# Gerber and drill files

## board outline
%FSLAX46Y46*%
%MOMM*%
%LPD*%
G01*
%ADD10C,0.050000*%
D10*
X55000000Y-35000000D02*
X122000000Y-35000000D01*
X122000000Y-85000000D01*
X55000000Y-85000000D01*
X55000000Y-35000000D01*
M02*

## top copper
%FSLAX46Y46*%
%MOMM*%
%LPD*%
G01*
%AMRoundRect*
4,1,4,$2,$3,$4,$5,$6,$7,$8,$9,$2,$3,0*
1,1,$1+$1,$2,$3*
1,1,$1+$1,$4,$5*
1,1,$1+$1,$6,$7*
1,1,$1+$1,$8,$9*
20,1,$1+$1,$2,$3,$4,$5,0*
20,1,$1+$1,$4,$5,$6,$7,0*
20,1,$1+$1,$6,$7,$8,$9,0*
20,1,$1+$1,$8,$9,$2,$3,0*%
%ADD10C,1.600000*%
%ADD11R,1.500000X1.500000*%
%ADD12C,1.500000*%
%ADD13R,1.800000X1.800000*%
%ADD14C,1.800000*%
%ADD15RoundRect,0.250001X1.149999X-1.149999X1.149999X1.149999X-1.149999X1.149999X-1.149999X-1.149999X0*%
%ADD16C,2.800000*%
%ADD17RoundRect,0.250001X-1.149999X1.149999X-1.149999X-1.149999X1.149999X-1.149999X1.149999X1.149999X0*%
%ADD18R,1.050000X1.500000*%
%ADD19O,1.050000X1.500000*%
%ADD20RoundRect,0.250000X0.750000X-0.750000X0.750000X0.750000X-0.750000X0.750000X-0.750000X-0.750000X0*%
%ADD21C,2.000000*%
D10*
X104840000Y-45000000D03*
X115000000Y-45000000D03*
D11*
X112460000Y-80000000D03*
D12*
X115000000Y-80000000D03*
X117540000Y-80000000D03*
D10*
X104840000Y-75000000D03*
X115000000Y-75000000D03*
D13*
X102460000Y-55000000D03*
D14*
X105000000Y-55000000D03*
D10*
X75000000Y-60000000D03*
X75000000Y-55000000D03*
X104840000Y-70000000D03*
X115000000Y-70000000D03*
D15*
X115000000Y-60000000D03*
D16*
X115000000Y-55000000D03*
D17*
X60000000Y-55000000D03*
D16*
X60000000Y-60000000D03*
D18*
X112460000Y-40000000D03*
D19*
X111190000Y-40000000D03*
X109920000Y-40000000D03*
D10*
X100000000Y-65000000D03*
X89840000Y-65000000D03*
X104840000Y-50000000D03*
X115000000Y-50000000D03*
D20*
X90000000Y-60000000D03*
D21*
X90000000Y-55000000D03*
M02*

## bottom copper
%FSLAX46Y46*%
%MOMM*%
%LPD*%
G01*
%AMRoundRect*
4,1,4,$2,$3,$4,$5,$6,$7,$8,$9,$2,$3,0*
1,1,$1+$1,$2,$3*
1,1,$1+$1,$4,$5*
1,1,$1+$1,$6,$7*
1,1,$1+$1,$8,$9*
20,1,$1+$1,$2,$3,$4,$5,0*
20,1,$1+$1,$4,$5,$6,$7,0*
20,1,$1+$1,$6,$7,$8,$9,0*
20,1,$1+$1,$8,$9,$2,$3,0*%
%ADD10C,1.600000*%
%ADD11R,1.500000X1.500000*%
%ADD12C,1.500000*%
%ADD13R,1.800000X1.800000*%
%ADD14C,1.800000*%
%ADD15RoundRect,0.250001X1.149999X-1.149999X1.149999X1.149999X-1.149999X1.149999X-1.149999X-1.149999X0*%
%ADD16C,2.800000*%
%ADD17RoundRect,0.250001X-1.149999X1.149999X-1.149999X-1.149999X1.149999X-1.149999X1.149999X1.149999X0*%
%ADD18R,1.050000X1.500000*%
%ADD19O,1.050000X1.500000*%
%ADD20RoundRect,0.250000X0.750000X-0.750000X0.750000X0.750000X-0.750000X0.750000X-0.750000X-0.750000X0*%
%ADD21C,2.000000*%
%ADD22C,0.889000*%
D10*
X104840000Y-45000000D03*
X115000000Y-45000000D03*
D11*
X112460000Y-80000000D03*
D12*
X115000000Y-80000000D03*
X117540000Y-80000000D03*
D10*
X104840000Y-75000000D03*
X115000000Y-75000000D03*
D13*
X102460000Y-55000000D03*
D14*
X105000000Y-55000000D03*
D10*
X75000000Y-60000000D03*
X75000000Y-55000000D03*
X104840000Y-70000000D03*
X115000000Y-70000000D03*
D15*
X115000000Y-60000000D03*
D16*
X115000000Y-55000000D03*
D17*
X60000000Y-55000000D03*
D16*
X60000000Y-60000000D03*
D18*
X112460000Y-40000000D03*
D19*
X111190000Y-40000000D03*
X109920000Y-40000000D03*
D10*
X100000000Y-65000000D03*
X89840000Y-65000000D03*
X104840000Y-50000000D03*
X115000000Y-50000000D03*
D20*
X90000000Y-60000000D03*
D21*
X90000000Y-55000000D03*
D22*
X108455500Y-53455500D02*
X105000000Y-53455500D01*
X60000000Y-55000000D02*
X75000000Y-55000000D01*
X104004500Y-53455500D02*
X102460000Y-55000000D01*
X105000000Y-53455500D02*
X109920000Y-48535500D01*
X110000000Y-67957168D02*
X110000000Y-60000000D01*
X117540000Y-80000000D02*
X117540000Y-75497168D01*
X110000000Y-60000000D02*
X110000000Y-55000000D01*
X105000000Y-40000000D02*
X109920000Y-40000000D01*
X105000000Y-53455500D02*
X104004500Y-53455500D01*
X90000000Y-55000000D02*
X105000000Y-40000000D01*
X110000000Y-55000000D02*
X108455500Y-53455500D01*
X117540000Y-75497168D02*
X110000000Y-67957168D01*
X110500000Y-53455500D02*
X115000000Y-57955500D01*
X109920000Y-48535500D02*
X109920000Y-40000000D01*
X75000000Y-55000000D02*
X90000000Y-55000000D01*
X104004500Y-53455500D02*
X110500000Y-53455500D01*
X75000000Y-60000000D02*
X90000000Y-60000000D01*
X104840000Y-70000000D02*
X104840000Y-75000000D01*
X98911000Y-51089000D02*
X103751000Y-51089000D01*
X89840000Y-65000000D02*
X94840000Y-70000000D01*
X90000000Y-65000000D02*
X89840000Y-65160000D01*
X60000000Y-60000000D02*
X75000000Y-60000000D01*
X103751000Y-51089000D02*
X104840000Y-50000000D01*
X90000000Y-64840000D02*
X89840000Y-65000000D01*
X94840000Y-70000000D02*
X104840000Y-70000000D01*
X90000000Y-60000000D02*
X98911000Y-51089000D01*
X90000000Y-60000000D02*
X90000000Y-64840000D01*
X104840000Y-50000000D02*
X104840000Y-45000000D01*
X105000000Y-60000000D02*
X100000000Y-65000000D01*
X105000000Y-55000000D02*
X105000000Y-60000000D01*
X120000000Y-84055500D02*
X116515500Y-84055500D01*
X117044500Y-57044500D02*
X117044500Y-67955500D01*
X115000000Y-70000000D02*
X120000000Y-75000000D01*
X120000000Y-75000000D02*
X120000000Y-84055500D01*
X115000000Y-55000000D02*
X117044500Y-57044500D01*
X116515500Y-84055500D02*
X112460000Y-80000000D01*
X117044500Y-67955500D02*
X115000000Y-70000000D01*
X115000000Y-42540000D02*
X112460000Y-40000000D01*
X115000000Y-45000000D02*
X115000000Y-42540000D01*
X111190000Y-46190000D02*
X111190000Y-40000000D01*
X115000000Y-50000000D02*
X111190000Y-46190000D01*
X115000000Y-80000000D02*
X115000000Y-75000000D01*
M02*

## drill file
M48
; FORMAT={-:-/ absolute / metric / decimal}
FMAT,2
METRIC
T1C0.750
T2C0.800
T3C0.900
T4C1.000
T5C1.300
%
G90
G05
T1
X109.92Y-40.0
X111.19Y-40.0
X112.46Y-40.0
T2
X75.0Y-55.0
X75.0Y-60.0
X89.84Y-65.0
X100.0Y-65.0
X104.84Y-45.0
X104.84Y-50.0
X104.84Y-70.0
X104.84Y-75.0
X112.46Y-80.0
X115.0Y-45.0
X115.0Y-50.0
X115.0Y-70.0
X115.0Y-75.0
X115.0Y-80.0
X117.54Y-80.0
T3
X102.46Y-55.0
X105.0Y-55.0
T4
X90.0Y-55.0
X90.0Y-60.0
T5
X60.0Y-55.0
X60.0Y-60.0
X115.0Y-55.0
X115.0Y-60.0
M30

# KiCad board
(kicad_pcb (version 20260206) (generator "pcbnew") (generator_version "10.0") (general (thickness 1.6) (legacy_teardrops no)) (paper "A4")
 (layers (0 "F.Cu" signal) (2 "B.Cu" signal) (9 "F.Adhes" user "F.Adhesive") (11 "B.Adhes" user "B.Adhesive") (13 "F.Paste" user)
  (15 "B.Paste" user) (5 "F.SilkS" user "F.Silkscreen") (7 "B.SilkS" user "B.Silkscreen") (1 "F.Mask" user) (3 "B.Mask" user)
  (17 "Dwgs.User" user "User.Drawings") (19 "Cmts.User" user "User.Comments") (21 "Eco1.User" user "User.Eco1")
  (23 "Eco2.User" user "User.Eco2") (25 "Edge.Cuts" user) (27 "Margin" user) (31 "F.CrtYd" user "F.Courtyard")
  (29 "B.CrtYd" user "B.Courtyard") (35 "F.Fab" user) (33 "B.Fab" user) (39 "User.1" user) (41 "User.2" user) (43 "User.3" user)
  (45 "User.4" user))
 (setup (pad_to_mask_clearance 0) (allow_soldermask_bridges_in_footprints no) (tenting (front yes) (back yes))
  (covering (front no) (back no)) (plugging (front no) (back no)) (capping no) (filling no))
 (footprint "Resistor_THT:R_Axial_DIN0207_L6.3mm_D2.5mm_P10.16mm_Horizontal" (layer "F.Cu") (at 104.84 45)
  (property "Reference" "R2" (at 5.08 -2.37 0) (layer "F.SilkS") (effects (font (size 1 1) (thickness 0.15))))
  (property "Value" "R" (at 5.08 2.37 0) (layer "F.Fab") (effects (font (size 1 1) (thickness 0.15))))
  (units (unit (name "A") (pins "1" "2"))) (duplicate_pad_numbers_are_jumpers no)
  (pad "1" thru_hole circle (at 0 0) (size 1.6 1.6) (drill 0.8) (layers "*.Cu" "*.Mask") (remove_unused_layers no) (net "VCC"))
  (pad "2" thru_hole circle (at 10.16 0) (size 1.6 1.6) (drill 0.8) (layers "*.Cu" "*.Mask") (remove_unused_layers no) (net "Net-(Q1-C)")))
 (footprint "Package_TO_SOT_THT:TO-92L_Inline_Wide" (layer "F.Cu") (at 112.46 80)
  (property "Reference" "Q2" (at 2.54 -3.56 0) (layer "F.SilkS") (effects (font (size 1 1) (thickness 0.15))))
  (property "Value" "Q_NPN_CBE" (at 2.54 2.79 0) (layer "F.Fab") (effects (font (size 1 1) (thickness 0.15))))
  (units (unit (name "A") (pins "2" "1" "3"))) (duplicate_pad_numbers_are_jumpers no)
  (pad "1" thru_hole rect (at 0 0) (size 1.5 1.5) (drill 0.8) (layers "*.Cu" "*.Mask") (remove_unused_layers no) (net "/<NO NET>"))
  (pad "2" thru_hole circle (at 2.54 0) (size 1.5 1.5) (drill 0.8) (layers "*.Cu" "*.Mask") (remove_unused_layers no) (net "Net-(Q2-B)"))
  (pad "3" thru_hole circle (at 5.08 0) (size 1.5 1.5) (drill 0.8) (layers "*.Cu" "*.Mask") (remove_unused_layers no) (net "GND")))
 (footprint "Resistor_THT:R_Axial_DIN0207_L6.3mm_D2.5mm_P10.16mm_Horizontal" (layer "F.Cu") (at 104.84 75)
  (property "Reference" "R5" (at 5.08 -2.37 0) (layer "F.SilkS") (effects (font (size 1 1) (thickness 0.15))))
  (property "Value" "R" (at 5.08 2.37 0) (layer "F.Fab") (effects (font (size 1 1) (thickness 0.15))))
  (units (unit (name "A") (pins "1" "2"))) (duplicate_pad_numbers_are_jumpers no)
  (pad "1" thru_hole circle (at 0 0) (size 1.6 1.6) (drill 0.8) (layers "*.Cu" "*.Mask") (remove_unused_layers no) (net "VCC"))
  (pad "2" thru_hole circle (at 10.16 0) (size 1.6 1.6) (drill 0.8) (layers "*.Cu" "*.Mask") (remove_unused_layers no) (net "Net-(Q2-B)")))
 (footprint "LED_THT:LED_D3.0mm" (layer "F.Cu") (at 102.46 55)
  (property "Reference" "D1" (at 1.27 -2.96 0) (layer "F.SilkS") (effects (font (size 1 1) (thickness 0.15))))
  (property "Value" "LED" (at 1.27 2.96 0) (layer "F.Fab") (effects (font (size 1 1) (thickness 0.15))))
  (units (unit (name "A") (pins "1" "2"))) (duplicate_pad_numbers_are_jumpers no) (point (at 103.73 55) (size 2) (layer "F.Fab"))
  (pad "1" thru_hole rect (at 0 0) (size 1.8 1.8) (drill 0.9) (layers "*.Cu" "*.Mask") (remove_unused_layers no) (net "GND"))
  (pad "2" thru_hole circle (at 2.54 0) (size 1.8 1.8) (drill 0.9) (layers "*.Cu" "*.Mask") (remove_unused_layers no) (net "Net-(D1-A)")))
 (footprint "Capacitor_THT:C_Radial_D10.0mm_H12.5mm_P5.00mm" (layer "F.Cu") (at 75 60 90)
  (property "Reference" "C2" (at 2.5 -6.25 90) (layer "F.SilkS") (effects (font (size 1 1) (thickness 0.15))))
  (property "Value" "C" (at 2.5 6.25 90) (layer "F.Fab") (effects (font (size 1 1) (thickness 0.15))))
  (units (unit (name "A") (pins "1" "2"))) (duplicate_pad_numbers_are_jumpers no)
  (pad "1" thru_hole circle (at 0 0 90) (size 1.6 1.6) (drill 0.8) (layers "*.Cu" "*.Mask") (remove_unused_layers no) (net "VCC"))
  (pad "2" thru_hole circle (at 5 0 90) (size 1.6 1.6) (drill 0.8) (layers "*.Cu" "*.Mask") (remove_unused_layers no) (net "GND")))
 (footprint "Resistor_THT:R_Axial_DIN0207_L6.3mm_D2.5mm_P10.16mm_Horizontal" (layer "F.Cu") (at 104.84 70)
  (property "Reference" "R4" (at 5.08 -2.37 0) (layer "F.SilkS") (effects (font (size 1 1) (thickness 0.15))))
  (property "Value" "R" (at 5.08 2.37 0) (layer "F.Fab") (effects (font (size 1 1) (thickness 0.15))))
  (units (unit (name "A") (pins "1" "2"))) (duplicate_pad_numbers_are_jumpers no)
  (pad "1" thru_hole circle (at 0 0) (size 1.6 1.6) (drill 0.8) (layers "*.Cu" "*.Mask") (remove_unused_layers no) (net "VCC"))
  (pad "2" thru_hole circle (at 10.16 0) (size 1.6 1.6) (drill 0.8) (layers "*.Cu" "*.Mask") (remove_unused_layers no) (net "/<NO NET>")))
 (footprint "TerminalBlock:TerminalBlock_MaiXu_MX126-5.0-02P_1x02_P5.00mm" (layer "F.Cu") (at 115 60 90)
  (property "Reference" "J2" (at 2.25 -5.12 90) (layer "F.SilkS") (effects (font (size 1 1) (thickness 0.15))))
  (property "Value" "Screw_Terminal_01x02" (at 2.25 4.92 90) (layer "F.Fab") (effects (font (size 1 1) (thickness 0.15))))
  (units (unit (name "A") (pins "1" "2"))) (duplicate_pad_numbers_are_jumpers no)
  (pad "1" thru_hole roundrect (at 0 0 90) (size 2.8 2.8) (drill 1.3) (layers "*.Cu" "*.Mask") (remove_unused_layers no)
   (roundrect_rratio 0.089286) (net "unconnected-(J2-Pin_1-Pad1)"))
  (pad "2" thru_hole circle (at 5 0 90) (size 2.8 2.8) (drill 1.3) (layers "*.Cu" "*.Mask") (remove_unused_layers no) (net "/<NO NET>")))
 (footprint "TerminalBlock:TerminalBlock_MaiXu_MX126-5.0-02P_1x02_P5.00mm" (layer "F.Cu") (at 60 55 -90)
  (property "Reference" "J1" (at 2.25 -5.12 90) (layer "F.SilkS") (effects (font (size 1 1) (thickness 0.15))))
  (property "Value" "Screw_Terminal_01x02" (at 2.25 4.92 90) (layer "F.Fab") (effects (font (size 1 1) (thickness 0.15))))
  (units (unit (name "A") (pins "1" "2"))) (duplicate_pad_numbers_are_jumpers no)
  (pad "1" thru_hole roundrect (at 0 0 270) (size 2.8 2.8) (drill 1.3) (layers "*.Cu" "*.Mask") (remove_unused_layers no)
   (roundrect_rratio 0.089286) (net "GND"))
  (pad "2" thru_hole circle (at 5 0 270) (size 2.8 2.8) (drill 1.3) (layers "*.Cu" "*.Mask") (remove_unused_layers no) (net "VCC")))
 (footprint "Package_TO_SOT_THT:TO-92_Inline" (layer "F.Cu") (at 112.46 40 180)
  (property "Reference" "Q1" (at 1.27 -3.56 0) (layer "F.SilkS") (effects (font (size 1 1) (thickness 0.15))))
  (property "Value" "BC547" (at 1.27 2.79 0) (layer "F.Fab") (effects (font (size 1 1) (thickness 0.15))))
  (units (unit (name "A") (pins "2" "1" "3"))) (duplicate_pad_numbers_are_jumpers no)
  (pad "1" thru_hole rect (at 0 0 180) (size 1.05 1.5) (drill 0.75) (layers "*.Cu" "*.Mask") (remove_unused_layers no) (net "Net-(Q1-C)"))
  (pad "2" thru_hole oval (at 1.27 0 180) (size 1.05 1.5) (drill 0.75) (layers "*.Cu" "*.Mask") (remove_unused_layers no) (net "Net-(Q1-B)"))
  (pad "3" thru_hole oval (at 2.54 0 180) (size 1.05 1.5) (drill 0.75) (layers "*.Cu" "*.Mask") (remove_unused_layers no) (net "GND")))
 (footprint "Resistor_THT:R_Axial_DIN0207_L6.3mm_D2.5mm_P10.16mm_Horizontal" (layer "F.Cu") (at 100 65 180)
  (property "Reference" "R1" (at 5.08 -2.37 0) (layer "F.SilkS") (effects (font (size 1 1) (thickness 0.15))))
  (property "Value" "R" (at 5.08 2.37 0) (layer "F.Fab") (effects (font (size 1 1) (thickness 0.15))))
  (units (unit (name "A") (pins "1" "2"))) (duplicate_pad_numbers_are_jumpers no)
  (pad "1" thru_hole circle (at 0 0 180) (size 1.6 1.6) (drill 0.8) (layers "*.Cu" "*.Mask") (remove_unused_layers no) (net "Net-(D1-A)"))
  (pad "2" thru_hole circle (at 10.16 0 180) (size 1.6 1.6) (drill 0.8) (layers "*.Cu" "*.Mask") (remove_unused_layers no) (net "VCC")))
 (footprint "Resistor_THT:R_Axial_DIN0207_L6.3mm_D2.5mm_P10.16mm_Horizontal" (layer "F.Cu") (at 104.84 50)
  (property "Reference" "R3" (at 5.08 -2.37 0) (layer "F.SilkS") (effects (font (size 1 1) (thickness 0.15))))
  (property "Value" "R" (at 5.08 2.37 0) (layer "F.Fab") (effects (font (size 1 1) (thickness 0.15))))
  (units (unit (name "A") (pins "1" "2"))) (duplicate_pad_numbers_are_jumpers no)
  (pad "1" thru_hole circle (at 0 0) (size 1.6 1.6) (drill 0.8) (layers "*.Cu" "*.Mask") (remove_unused_layers no) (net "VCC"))
  (pad "2" thru_hole circle (at 10.16 0) (size 1.6 1.6) (drill 0.8) (layers "*.Cu" "*.Mask") (remove_unused_layers no) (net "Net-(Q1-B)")))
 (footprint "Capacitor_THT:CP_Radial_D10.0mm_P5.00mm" (layer "F.Cu") (at 90 60 90)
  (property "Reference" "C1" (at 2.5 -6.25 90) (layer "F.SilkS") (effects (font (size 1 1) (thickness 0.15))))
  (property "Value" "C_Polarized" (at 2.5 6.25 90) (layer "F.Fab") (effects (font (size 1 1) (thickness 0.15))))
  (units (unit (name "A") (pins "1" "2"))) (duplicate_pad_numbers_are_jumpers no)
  (pad "1" thru_hole roundrect (at 0 0 90) (size 2 2) (drill 1) (layers "*.Cu" "*.Mask") (remove_unused_layers no) (roundrect_rratio 0.125)
   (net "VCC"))
  (pad "2" thru_hole circle (at 5 0 90) (size 2 2) (drill 1) (layers "*.Cu" "*.Mask") (remove_unused_layers no) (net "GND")))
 (gr_rect (start 55 35) (end 122 85) (stroke (width 0.05) (type default)) (fill no) (layer "Edge.Cuts"))
 (segment (start 108.4555 53.4555) (end 105 53.4555) (width 0.889) (layer "B.Cu") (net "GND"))
 (segment (start 60 55) (end 75 55) (width 0.889) (layer "B.Cu") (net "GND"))
 (segment (start 104.0045 53.4555) (end 102.46 55) (width 0.889) (layer "B.Cu") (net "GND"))
 (segment (start 105 53.4555) (end 109.92 48.5355) (width 0.889) (layer "B.Cu") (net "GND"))
 (segment (start 110 67.957168) (end 110 60) (width 0.889) (layer "B.Cu") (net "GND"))
 (segment (start 117.54 80) (end 117.54 75.497168) (width 0.889) (layer "B.Cu") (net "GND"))
 (segment (start 110 60) (end 110 55) (width 0.889) (layer "B.Cu") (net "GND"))
 (segment (start 105 40) (end 109.92 40) (width 0.889) (layer "B.Cu") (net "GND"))
 (segment (start 105 53.4555) (end 104.0045 53.4555) (width 0.889) (layer "B.Cu") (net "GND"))
 (segment (start 90 55) (end 105 40) (width 0.889) (layer "B.Cu") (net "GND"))
 (segment (start 110 55) (end 108.4555 53.4555) (width 0.889) (layer "B.Cu") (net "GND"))
 (segment (start 117.54 75.497168) (end 110 67.957168) (width 0.889) (layer "B.Cu") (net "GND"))
 (segment (start 110.5 53.4555) (end 115 57.9555) (width 0.889) (layer "B.Cu") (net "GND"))
 (segment (start 109.92 48.5355) (end 109.92 40) (width 0.889) (layer "B.Cu") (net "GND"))
 (segment (start 75 55) (end 90 55) (width 0.889) (layer "B.Cu") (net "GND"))
 (segment (start 104.0045 53.4555) (end 110.5 53.4555) (width 0.889) (layer "B.Cu") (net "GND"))
 (segment (start 75 60) (end 90 60) (width 0.889) (layer "B.Cu") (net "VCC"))
 (segment (start 104.84 70) (end 104.84 75) (width 0.889) (layer "B.Cu") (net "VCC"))
 (segment (start 98.911 51.089) (end 103.751 51.089) (width 0.889) (layer "B.Cu") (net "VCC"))
 (segment (start 89.84 65) (end 94.84 70) (width 0.889) (layer "B.Cu") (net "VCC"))
 (segment (start 90 65) (end 89.84 65.16) (width 0.889) (layer "B.Cu") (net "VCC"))
 (segment (start 60 60) (end 75 60) (width 0.889) (layer "B.Cu") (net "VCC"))
 (segment (start 103.751 51.089) (end 104.84 50) (width 0.889) (layer "B.Cu") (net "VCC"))
 (segment (start 90 64.84) (end 89.84 65) (width 0.889) (layer "B.Cu") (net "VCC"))
 (segment (start 94.84 70) (end 104.84 70) (width 0.889) (layer "B.Cu") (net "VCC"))
 (segment (start 90 60) (end 98.911 51.089) (width 0.889) (layer "B.Cu") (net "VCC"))
 (segment (start 90 60) (end 90 64.84) (width 0.889) (layer "B.Cu") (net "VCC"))
 (segment (start 104.84 50) (end 104.84 45) (width 0.889) (layer "B.Cu") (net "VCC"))
 (segment (start 105 60) (end 100 65) (width 0.889) (layer "B.Cu") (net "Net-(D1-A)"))
 (segment (start 105 55) (end 105 60) (width 0.889) (layer "B.Cu") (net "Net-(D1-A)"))
 (segment (start 120 84.0555) (end 116.5155 84.0555) (width 0.889) (layer "B.Cu") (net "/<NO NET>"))
 (segment (start 117.0445 57.0445) (end 117.0445 67.9555) (width 0.889) (layer "B.Cu") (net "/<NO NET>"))
 (segment (start 115 70) (end 120 75) (width 0.889) (layer "B.Cu") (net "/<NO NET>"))
 (segment (start 120 75) (end 120 84.0555) (width 0.889) (layer "B.Cu") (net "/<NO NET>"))
 (segment (start 115 55) (end 117.0445 57.0445) (width 0.889) (layer "B.Cu") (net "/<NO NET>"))
 (segment (start 116.5155 84.0555) (end 112.46 80) (width 0.889) (layer "B.Cu") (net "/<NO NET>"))
 (segment (start 117.0445 67.9555) (end 115 70) (width 0.889) (layer "B.Cu") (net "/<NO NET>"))
 (segment (start 115 42.54) (end 112.46 40) (width 0.889) (layer "B.Cu") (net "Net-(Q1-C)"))
 (segment (start 115 45) (end 115 42.54) (width 0.889) (layer "B.Cu") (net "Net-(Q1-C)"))
 (segment (start 111.19 46.19) (end 111.19 40) (width 0.889) (layer "B.Cu") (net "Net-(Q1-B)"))
 (segment (start 115 50) (end 111.19 46.19) (width 0.889) (layer "B.Cu") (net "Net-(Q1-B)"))
 (segment (start 115 80) (end 115 75) (width 0.889) (layer "B.Cu") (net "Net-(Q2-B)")))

